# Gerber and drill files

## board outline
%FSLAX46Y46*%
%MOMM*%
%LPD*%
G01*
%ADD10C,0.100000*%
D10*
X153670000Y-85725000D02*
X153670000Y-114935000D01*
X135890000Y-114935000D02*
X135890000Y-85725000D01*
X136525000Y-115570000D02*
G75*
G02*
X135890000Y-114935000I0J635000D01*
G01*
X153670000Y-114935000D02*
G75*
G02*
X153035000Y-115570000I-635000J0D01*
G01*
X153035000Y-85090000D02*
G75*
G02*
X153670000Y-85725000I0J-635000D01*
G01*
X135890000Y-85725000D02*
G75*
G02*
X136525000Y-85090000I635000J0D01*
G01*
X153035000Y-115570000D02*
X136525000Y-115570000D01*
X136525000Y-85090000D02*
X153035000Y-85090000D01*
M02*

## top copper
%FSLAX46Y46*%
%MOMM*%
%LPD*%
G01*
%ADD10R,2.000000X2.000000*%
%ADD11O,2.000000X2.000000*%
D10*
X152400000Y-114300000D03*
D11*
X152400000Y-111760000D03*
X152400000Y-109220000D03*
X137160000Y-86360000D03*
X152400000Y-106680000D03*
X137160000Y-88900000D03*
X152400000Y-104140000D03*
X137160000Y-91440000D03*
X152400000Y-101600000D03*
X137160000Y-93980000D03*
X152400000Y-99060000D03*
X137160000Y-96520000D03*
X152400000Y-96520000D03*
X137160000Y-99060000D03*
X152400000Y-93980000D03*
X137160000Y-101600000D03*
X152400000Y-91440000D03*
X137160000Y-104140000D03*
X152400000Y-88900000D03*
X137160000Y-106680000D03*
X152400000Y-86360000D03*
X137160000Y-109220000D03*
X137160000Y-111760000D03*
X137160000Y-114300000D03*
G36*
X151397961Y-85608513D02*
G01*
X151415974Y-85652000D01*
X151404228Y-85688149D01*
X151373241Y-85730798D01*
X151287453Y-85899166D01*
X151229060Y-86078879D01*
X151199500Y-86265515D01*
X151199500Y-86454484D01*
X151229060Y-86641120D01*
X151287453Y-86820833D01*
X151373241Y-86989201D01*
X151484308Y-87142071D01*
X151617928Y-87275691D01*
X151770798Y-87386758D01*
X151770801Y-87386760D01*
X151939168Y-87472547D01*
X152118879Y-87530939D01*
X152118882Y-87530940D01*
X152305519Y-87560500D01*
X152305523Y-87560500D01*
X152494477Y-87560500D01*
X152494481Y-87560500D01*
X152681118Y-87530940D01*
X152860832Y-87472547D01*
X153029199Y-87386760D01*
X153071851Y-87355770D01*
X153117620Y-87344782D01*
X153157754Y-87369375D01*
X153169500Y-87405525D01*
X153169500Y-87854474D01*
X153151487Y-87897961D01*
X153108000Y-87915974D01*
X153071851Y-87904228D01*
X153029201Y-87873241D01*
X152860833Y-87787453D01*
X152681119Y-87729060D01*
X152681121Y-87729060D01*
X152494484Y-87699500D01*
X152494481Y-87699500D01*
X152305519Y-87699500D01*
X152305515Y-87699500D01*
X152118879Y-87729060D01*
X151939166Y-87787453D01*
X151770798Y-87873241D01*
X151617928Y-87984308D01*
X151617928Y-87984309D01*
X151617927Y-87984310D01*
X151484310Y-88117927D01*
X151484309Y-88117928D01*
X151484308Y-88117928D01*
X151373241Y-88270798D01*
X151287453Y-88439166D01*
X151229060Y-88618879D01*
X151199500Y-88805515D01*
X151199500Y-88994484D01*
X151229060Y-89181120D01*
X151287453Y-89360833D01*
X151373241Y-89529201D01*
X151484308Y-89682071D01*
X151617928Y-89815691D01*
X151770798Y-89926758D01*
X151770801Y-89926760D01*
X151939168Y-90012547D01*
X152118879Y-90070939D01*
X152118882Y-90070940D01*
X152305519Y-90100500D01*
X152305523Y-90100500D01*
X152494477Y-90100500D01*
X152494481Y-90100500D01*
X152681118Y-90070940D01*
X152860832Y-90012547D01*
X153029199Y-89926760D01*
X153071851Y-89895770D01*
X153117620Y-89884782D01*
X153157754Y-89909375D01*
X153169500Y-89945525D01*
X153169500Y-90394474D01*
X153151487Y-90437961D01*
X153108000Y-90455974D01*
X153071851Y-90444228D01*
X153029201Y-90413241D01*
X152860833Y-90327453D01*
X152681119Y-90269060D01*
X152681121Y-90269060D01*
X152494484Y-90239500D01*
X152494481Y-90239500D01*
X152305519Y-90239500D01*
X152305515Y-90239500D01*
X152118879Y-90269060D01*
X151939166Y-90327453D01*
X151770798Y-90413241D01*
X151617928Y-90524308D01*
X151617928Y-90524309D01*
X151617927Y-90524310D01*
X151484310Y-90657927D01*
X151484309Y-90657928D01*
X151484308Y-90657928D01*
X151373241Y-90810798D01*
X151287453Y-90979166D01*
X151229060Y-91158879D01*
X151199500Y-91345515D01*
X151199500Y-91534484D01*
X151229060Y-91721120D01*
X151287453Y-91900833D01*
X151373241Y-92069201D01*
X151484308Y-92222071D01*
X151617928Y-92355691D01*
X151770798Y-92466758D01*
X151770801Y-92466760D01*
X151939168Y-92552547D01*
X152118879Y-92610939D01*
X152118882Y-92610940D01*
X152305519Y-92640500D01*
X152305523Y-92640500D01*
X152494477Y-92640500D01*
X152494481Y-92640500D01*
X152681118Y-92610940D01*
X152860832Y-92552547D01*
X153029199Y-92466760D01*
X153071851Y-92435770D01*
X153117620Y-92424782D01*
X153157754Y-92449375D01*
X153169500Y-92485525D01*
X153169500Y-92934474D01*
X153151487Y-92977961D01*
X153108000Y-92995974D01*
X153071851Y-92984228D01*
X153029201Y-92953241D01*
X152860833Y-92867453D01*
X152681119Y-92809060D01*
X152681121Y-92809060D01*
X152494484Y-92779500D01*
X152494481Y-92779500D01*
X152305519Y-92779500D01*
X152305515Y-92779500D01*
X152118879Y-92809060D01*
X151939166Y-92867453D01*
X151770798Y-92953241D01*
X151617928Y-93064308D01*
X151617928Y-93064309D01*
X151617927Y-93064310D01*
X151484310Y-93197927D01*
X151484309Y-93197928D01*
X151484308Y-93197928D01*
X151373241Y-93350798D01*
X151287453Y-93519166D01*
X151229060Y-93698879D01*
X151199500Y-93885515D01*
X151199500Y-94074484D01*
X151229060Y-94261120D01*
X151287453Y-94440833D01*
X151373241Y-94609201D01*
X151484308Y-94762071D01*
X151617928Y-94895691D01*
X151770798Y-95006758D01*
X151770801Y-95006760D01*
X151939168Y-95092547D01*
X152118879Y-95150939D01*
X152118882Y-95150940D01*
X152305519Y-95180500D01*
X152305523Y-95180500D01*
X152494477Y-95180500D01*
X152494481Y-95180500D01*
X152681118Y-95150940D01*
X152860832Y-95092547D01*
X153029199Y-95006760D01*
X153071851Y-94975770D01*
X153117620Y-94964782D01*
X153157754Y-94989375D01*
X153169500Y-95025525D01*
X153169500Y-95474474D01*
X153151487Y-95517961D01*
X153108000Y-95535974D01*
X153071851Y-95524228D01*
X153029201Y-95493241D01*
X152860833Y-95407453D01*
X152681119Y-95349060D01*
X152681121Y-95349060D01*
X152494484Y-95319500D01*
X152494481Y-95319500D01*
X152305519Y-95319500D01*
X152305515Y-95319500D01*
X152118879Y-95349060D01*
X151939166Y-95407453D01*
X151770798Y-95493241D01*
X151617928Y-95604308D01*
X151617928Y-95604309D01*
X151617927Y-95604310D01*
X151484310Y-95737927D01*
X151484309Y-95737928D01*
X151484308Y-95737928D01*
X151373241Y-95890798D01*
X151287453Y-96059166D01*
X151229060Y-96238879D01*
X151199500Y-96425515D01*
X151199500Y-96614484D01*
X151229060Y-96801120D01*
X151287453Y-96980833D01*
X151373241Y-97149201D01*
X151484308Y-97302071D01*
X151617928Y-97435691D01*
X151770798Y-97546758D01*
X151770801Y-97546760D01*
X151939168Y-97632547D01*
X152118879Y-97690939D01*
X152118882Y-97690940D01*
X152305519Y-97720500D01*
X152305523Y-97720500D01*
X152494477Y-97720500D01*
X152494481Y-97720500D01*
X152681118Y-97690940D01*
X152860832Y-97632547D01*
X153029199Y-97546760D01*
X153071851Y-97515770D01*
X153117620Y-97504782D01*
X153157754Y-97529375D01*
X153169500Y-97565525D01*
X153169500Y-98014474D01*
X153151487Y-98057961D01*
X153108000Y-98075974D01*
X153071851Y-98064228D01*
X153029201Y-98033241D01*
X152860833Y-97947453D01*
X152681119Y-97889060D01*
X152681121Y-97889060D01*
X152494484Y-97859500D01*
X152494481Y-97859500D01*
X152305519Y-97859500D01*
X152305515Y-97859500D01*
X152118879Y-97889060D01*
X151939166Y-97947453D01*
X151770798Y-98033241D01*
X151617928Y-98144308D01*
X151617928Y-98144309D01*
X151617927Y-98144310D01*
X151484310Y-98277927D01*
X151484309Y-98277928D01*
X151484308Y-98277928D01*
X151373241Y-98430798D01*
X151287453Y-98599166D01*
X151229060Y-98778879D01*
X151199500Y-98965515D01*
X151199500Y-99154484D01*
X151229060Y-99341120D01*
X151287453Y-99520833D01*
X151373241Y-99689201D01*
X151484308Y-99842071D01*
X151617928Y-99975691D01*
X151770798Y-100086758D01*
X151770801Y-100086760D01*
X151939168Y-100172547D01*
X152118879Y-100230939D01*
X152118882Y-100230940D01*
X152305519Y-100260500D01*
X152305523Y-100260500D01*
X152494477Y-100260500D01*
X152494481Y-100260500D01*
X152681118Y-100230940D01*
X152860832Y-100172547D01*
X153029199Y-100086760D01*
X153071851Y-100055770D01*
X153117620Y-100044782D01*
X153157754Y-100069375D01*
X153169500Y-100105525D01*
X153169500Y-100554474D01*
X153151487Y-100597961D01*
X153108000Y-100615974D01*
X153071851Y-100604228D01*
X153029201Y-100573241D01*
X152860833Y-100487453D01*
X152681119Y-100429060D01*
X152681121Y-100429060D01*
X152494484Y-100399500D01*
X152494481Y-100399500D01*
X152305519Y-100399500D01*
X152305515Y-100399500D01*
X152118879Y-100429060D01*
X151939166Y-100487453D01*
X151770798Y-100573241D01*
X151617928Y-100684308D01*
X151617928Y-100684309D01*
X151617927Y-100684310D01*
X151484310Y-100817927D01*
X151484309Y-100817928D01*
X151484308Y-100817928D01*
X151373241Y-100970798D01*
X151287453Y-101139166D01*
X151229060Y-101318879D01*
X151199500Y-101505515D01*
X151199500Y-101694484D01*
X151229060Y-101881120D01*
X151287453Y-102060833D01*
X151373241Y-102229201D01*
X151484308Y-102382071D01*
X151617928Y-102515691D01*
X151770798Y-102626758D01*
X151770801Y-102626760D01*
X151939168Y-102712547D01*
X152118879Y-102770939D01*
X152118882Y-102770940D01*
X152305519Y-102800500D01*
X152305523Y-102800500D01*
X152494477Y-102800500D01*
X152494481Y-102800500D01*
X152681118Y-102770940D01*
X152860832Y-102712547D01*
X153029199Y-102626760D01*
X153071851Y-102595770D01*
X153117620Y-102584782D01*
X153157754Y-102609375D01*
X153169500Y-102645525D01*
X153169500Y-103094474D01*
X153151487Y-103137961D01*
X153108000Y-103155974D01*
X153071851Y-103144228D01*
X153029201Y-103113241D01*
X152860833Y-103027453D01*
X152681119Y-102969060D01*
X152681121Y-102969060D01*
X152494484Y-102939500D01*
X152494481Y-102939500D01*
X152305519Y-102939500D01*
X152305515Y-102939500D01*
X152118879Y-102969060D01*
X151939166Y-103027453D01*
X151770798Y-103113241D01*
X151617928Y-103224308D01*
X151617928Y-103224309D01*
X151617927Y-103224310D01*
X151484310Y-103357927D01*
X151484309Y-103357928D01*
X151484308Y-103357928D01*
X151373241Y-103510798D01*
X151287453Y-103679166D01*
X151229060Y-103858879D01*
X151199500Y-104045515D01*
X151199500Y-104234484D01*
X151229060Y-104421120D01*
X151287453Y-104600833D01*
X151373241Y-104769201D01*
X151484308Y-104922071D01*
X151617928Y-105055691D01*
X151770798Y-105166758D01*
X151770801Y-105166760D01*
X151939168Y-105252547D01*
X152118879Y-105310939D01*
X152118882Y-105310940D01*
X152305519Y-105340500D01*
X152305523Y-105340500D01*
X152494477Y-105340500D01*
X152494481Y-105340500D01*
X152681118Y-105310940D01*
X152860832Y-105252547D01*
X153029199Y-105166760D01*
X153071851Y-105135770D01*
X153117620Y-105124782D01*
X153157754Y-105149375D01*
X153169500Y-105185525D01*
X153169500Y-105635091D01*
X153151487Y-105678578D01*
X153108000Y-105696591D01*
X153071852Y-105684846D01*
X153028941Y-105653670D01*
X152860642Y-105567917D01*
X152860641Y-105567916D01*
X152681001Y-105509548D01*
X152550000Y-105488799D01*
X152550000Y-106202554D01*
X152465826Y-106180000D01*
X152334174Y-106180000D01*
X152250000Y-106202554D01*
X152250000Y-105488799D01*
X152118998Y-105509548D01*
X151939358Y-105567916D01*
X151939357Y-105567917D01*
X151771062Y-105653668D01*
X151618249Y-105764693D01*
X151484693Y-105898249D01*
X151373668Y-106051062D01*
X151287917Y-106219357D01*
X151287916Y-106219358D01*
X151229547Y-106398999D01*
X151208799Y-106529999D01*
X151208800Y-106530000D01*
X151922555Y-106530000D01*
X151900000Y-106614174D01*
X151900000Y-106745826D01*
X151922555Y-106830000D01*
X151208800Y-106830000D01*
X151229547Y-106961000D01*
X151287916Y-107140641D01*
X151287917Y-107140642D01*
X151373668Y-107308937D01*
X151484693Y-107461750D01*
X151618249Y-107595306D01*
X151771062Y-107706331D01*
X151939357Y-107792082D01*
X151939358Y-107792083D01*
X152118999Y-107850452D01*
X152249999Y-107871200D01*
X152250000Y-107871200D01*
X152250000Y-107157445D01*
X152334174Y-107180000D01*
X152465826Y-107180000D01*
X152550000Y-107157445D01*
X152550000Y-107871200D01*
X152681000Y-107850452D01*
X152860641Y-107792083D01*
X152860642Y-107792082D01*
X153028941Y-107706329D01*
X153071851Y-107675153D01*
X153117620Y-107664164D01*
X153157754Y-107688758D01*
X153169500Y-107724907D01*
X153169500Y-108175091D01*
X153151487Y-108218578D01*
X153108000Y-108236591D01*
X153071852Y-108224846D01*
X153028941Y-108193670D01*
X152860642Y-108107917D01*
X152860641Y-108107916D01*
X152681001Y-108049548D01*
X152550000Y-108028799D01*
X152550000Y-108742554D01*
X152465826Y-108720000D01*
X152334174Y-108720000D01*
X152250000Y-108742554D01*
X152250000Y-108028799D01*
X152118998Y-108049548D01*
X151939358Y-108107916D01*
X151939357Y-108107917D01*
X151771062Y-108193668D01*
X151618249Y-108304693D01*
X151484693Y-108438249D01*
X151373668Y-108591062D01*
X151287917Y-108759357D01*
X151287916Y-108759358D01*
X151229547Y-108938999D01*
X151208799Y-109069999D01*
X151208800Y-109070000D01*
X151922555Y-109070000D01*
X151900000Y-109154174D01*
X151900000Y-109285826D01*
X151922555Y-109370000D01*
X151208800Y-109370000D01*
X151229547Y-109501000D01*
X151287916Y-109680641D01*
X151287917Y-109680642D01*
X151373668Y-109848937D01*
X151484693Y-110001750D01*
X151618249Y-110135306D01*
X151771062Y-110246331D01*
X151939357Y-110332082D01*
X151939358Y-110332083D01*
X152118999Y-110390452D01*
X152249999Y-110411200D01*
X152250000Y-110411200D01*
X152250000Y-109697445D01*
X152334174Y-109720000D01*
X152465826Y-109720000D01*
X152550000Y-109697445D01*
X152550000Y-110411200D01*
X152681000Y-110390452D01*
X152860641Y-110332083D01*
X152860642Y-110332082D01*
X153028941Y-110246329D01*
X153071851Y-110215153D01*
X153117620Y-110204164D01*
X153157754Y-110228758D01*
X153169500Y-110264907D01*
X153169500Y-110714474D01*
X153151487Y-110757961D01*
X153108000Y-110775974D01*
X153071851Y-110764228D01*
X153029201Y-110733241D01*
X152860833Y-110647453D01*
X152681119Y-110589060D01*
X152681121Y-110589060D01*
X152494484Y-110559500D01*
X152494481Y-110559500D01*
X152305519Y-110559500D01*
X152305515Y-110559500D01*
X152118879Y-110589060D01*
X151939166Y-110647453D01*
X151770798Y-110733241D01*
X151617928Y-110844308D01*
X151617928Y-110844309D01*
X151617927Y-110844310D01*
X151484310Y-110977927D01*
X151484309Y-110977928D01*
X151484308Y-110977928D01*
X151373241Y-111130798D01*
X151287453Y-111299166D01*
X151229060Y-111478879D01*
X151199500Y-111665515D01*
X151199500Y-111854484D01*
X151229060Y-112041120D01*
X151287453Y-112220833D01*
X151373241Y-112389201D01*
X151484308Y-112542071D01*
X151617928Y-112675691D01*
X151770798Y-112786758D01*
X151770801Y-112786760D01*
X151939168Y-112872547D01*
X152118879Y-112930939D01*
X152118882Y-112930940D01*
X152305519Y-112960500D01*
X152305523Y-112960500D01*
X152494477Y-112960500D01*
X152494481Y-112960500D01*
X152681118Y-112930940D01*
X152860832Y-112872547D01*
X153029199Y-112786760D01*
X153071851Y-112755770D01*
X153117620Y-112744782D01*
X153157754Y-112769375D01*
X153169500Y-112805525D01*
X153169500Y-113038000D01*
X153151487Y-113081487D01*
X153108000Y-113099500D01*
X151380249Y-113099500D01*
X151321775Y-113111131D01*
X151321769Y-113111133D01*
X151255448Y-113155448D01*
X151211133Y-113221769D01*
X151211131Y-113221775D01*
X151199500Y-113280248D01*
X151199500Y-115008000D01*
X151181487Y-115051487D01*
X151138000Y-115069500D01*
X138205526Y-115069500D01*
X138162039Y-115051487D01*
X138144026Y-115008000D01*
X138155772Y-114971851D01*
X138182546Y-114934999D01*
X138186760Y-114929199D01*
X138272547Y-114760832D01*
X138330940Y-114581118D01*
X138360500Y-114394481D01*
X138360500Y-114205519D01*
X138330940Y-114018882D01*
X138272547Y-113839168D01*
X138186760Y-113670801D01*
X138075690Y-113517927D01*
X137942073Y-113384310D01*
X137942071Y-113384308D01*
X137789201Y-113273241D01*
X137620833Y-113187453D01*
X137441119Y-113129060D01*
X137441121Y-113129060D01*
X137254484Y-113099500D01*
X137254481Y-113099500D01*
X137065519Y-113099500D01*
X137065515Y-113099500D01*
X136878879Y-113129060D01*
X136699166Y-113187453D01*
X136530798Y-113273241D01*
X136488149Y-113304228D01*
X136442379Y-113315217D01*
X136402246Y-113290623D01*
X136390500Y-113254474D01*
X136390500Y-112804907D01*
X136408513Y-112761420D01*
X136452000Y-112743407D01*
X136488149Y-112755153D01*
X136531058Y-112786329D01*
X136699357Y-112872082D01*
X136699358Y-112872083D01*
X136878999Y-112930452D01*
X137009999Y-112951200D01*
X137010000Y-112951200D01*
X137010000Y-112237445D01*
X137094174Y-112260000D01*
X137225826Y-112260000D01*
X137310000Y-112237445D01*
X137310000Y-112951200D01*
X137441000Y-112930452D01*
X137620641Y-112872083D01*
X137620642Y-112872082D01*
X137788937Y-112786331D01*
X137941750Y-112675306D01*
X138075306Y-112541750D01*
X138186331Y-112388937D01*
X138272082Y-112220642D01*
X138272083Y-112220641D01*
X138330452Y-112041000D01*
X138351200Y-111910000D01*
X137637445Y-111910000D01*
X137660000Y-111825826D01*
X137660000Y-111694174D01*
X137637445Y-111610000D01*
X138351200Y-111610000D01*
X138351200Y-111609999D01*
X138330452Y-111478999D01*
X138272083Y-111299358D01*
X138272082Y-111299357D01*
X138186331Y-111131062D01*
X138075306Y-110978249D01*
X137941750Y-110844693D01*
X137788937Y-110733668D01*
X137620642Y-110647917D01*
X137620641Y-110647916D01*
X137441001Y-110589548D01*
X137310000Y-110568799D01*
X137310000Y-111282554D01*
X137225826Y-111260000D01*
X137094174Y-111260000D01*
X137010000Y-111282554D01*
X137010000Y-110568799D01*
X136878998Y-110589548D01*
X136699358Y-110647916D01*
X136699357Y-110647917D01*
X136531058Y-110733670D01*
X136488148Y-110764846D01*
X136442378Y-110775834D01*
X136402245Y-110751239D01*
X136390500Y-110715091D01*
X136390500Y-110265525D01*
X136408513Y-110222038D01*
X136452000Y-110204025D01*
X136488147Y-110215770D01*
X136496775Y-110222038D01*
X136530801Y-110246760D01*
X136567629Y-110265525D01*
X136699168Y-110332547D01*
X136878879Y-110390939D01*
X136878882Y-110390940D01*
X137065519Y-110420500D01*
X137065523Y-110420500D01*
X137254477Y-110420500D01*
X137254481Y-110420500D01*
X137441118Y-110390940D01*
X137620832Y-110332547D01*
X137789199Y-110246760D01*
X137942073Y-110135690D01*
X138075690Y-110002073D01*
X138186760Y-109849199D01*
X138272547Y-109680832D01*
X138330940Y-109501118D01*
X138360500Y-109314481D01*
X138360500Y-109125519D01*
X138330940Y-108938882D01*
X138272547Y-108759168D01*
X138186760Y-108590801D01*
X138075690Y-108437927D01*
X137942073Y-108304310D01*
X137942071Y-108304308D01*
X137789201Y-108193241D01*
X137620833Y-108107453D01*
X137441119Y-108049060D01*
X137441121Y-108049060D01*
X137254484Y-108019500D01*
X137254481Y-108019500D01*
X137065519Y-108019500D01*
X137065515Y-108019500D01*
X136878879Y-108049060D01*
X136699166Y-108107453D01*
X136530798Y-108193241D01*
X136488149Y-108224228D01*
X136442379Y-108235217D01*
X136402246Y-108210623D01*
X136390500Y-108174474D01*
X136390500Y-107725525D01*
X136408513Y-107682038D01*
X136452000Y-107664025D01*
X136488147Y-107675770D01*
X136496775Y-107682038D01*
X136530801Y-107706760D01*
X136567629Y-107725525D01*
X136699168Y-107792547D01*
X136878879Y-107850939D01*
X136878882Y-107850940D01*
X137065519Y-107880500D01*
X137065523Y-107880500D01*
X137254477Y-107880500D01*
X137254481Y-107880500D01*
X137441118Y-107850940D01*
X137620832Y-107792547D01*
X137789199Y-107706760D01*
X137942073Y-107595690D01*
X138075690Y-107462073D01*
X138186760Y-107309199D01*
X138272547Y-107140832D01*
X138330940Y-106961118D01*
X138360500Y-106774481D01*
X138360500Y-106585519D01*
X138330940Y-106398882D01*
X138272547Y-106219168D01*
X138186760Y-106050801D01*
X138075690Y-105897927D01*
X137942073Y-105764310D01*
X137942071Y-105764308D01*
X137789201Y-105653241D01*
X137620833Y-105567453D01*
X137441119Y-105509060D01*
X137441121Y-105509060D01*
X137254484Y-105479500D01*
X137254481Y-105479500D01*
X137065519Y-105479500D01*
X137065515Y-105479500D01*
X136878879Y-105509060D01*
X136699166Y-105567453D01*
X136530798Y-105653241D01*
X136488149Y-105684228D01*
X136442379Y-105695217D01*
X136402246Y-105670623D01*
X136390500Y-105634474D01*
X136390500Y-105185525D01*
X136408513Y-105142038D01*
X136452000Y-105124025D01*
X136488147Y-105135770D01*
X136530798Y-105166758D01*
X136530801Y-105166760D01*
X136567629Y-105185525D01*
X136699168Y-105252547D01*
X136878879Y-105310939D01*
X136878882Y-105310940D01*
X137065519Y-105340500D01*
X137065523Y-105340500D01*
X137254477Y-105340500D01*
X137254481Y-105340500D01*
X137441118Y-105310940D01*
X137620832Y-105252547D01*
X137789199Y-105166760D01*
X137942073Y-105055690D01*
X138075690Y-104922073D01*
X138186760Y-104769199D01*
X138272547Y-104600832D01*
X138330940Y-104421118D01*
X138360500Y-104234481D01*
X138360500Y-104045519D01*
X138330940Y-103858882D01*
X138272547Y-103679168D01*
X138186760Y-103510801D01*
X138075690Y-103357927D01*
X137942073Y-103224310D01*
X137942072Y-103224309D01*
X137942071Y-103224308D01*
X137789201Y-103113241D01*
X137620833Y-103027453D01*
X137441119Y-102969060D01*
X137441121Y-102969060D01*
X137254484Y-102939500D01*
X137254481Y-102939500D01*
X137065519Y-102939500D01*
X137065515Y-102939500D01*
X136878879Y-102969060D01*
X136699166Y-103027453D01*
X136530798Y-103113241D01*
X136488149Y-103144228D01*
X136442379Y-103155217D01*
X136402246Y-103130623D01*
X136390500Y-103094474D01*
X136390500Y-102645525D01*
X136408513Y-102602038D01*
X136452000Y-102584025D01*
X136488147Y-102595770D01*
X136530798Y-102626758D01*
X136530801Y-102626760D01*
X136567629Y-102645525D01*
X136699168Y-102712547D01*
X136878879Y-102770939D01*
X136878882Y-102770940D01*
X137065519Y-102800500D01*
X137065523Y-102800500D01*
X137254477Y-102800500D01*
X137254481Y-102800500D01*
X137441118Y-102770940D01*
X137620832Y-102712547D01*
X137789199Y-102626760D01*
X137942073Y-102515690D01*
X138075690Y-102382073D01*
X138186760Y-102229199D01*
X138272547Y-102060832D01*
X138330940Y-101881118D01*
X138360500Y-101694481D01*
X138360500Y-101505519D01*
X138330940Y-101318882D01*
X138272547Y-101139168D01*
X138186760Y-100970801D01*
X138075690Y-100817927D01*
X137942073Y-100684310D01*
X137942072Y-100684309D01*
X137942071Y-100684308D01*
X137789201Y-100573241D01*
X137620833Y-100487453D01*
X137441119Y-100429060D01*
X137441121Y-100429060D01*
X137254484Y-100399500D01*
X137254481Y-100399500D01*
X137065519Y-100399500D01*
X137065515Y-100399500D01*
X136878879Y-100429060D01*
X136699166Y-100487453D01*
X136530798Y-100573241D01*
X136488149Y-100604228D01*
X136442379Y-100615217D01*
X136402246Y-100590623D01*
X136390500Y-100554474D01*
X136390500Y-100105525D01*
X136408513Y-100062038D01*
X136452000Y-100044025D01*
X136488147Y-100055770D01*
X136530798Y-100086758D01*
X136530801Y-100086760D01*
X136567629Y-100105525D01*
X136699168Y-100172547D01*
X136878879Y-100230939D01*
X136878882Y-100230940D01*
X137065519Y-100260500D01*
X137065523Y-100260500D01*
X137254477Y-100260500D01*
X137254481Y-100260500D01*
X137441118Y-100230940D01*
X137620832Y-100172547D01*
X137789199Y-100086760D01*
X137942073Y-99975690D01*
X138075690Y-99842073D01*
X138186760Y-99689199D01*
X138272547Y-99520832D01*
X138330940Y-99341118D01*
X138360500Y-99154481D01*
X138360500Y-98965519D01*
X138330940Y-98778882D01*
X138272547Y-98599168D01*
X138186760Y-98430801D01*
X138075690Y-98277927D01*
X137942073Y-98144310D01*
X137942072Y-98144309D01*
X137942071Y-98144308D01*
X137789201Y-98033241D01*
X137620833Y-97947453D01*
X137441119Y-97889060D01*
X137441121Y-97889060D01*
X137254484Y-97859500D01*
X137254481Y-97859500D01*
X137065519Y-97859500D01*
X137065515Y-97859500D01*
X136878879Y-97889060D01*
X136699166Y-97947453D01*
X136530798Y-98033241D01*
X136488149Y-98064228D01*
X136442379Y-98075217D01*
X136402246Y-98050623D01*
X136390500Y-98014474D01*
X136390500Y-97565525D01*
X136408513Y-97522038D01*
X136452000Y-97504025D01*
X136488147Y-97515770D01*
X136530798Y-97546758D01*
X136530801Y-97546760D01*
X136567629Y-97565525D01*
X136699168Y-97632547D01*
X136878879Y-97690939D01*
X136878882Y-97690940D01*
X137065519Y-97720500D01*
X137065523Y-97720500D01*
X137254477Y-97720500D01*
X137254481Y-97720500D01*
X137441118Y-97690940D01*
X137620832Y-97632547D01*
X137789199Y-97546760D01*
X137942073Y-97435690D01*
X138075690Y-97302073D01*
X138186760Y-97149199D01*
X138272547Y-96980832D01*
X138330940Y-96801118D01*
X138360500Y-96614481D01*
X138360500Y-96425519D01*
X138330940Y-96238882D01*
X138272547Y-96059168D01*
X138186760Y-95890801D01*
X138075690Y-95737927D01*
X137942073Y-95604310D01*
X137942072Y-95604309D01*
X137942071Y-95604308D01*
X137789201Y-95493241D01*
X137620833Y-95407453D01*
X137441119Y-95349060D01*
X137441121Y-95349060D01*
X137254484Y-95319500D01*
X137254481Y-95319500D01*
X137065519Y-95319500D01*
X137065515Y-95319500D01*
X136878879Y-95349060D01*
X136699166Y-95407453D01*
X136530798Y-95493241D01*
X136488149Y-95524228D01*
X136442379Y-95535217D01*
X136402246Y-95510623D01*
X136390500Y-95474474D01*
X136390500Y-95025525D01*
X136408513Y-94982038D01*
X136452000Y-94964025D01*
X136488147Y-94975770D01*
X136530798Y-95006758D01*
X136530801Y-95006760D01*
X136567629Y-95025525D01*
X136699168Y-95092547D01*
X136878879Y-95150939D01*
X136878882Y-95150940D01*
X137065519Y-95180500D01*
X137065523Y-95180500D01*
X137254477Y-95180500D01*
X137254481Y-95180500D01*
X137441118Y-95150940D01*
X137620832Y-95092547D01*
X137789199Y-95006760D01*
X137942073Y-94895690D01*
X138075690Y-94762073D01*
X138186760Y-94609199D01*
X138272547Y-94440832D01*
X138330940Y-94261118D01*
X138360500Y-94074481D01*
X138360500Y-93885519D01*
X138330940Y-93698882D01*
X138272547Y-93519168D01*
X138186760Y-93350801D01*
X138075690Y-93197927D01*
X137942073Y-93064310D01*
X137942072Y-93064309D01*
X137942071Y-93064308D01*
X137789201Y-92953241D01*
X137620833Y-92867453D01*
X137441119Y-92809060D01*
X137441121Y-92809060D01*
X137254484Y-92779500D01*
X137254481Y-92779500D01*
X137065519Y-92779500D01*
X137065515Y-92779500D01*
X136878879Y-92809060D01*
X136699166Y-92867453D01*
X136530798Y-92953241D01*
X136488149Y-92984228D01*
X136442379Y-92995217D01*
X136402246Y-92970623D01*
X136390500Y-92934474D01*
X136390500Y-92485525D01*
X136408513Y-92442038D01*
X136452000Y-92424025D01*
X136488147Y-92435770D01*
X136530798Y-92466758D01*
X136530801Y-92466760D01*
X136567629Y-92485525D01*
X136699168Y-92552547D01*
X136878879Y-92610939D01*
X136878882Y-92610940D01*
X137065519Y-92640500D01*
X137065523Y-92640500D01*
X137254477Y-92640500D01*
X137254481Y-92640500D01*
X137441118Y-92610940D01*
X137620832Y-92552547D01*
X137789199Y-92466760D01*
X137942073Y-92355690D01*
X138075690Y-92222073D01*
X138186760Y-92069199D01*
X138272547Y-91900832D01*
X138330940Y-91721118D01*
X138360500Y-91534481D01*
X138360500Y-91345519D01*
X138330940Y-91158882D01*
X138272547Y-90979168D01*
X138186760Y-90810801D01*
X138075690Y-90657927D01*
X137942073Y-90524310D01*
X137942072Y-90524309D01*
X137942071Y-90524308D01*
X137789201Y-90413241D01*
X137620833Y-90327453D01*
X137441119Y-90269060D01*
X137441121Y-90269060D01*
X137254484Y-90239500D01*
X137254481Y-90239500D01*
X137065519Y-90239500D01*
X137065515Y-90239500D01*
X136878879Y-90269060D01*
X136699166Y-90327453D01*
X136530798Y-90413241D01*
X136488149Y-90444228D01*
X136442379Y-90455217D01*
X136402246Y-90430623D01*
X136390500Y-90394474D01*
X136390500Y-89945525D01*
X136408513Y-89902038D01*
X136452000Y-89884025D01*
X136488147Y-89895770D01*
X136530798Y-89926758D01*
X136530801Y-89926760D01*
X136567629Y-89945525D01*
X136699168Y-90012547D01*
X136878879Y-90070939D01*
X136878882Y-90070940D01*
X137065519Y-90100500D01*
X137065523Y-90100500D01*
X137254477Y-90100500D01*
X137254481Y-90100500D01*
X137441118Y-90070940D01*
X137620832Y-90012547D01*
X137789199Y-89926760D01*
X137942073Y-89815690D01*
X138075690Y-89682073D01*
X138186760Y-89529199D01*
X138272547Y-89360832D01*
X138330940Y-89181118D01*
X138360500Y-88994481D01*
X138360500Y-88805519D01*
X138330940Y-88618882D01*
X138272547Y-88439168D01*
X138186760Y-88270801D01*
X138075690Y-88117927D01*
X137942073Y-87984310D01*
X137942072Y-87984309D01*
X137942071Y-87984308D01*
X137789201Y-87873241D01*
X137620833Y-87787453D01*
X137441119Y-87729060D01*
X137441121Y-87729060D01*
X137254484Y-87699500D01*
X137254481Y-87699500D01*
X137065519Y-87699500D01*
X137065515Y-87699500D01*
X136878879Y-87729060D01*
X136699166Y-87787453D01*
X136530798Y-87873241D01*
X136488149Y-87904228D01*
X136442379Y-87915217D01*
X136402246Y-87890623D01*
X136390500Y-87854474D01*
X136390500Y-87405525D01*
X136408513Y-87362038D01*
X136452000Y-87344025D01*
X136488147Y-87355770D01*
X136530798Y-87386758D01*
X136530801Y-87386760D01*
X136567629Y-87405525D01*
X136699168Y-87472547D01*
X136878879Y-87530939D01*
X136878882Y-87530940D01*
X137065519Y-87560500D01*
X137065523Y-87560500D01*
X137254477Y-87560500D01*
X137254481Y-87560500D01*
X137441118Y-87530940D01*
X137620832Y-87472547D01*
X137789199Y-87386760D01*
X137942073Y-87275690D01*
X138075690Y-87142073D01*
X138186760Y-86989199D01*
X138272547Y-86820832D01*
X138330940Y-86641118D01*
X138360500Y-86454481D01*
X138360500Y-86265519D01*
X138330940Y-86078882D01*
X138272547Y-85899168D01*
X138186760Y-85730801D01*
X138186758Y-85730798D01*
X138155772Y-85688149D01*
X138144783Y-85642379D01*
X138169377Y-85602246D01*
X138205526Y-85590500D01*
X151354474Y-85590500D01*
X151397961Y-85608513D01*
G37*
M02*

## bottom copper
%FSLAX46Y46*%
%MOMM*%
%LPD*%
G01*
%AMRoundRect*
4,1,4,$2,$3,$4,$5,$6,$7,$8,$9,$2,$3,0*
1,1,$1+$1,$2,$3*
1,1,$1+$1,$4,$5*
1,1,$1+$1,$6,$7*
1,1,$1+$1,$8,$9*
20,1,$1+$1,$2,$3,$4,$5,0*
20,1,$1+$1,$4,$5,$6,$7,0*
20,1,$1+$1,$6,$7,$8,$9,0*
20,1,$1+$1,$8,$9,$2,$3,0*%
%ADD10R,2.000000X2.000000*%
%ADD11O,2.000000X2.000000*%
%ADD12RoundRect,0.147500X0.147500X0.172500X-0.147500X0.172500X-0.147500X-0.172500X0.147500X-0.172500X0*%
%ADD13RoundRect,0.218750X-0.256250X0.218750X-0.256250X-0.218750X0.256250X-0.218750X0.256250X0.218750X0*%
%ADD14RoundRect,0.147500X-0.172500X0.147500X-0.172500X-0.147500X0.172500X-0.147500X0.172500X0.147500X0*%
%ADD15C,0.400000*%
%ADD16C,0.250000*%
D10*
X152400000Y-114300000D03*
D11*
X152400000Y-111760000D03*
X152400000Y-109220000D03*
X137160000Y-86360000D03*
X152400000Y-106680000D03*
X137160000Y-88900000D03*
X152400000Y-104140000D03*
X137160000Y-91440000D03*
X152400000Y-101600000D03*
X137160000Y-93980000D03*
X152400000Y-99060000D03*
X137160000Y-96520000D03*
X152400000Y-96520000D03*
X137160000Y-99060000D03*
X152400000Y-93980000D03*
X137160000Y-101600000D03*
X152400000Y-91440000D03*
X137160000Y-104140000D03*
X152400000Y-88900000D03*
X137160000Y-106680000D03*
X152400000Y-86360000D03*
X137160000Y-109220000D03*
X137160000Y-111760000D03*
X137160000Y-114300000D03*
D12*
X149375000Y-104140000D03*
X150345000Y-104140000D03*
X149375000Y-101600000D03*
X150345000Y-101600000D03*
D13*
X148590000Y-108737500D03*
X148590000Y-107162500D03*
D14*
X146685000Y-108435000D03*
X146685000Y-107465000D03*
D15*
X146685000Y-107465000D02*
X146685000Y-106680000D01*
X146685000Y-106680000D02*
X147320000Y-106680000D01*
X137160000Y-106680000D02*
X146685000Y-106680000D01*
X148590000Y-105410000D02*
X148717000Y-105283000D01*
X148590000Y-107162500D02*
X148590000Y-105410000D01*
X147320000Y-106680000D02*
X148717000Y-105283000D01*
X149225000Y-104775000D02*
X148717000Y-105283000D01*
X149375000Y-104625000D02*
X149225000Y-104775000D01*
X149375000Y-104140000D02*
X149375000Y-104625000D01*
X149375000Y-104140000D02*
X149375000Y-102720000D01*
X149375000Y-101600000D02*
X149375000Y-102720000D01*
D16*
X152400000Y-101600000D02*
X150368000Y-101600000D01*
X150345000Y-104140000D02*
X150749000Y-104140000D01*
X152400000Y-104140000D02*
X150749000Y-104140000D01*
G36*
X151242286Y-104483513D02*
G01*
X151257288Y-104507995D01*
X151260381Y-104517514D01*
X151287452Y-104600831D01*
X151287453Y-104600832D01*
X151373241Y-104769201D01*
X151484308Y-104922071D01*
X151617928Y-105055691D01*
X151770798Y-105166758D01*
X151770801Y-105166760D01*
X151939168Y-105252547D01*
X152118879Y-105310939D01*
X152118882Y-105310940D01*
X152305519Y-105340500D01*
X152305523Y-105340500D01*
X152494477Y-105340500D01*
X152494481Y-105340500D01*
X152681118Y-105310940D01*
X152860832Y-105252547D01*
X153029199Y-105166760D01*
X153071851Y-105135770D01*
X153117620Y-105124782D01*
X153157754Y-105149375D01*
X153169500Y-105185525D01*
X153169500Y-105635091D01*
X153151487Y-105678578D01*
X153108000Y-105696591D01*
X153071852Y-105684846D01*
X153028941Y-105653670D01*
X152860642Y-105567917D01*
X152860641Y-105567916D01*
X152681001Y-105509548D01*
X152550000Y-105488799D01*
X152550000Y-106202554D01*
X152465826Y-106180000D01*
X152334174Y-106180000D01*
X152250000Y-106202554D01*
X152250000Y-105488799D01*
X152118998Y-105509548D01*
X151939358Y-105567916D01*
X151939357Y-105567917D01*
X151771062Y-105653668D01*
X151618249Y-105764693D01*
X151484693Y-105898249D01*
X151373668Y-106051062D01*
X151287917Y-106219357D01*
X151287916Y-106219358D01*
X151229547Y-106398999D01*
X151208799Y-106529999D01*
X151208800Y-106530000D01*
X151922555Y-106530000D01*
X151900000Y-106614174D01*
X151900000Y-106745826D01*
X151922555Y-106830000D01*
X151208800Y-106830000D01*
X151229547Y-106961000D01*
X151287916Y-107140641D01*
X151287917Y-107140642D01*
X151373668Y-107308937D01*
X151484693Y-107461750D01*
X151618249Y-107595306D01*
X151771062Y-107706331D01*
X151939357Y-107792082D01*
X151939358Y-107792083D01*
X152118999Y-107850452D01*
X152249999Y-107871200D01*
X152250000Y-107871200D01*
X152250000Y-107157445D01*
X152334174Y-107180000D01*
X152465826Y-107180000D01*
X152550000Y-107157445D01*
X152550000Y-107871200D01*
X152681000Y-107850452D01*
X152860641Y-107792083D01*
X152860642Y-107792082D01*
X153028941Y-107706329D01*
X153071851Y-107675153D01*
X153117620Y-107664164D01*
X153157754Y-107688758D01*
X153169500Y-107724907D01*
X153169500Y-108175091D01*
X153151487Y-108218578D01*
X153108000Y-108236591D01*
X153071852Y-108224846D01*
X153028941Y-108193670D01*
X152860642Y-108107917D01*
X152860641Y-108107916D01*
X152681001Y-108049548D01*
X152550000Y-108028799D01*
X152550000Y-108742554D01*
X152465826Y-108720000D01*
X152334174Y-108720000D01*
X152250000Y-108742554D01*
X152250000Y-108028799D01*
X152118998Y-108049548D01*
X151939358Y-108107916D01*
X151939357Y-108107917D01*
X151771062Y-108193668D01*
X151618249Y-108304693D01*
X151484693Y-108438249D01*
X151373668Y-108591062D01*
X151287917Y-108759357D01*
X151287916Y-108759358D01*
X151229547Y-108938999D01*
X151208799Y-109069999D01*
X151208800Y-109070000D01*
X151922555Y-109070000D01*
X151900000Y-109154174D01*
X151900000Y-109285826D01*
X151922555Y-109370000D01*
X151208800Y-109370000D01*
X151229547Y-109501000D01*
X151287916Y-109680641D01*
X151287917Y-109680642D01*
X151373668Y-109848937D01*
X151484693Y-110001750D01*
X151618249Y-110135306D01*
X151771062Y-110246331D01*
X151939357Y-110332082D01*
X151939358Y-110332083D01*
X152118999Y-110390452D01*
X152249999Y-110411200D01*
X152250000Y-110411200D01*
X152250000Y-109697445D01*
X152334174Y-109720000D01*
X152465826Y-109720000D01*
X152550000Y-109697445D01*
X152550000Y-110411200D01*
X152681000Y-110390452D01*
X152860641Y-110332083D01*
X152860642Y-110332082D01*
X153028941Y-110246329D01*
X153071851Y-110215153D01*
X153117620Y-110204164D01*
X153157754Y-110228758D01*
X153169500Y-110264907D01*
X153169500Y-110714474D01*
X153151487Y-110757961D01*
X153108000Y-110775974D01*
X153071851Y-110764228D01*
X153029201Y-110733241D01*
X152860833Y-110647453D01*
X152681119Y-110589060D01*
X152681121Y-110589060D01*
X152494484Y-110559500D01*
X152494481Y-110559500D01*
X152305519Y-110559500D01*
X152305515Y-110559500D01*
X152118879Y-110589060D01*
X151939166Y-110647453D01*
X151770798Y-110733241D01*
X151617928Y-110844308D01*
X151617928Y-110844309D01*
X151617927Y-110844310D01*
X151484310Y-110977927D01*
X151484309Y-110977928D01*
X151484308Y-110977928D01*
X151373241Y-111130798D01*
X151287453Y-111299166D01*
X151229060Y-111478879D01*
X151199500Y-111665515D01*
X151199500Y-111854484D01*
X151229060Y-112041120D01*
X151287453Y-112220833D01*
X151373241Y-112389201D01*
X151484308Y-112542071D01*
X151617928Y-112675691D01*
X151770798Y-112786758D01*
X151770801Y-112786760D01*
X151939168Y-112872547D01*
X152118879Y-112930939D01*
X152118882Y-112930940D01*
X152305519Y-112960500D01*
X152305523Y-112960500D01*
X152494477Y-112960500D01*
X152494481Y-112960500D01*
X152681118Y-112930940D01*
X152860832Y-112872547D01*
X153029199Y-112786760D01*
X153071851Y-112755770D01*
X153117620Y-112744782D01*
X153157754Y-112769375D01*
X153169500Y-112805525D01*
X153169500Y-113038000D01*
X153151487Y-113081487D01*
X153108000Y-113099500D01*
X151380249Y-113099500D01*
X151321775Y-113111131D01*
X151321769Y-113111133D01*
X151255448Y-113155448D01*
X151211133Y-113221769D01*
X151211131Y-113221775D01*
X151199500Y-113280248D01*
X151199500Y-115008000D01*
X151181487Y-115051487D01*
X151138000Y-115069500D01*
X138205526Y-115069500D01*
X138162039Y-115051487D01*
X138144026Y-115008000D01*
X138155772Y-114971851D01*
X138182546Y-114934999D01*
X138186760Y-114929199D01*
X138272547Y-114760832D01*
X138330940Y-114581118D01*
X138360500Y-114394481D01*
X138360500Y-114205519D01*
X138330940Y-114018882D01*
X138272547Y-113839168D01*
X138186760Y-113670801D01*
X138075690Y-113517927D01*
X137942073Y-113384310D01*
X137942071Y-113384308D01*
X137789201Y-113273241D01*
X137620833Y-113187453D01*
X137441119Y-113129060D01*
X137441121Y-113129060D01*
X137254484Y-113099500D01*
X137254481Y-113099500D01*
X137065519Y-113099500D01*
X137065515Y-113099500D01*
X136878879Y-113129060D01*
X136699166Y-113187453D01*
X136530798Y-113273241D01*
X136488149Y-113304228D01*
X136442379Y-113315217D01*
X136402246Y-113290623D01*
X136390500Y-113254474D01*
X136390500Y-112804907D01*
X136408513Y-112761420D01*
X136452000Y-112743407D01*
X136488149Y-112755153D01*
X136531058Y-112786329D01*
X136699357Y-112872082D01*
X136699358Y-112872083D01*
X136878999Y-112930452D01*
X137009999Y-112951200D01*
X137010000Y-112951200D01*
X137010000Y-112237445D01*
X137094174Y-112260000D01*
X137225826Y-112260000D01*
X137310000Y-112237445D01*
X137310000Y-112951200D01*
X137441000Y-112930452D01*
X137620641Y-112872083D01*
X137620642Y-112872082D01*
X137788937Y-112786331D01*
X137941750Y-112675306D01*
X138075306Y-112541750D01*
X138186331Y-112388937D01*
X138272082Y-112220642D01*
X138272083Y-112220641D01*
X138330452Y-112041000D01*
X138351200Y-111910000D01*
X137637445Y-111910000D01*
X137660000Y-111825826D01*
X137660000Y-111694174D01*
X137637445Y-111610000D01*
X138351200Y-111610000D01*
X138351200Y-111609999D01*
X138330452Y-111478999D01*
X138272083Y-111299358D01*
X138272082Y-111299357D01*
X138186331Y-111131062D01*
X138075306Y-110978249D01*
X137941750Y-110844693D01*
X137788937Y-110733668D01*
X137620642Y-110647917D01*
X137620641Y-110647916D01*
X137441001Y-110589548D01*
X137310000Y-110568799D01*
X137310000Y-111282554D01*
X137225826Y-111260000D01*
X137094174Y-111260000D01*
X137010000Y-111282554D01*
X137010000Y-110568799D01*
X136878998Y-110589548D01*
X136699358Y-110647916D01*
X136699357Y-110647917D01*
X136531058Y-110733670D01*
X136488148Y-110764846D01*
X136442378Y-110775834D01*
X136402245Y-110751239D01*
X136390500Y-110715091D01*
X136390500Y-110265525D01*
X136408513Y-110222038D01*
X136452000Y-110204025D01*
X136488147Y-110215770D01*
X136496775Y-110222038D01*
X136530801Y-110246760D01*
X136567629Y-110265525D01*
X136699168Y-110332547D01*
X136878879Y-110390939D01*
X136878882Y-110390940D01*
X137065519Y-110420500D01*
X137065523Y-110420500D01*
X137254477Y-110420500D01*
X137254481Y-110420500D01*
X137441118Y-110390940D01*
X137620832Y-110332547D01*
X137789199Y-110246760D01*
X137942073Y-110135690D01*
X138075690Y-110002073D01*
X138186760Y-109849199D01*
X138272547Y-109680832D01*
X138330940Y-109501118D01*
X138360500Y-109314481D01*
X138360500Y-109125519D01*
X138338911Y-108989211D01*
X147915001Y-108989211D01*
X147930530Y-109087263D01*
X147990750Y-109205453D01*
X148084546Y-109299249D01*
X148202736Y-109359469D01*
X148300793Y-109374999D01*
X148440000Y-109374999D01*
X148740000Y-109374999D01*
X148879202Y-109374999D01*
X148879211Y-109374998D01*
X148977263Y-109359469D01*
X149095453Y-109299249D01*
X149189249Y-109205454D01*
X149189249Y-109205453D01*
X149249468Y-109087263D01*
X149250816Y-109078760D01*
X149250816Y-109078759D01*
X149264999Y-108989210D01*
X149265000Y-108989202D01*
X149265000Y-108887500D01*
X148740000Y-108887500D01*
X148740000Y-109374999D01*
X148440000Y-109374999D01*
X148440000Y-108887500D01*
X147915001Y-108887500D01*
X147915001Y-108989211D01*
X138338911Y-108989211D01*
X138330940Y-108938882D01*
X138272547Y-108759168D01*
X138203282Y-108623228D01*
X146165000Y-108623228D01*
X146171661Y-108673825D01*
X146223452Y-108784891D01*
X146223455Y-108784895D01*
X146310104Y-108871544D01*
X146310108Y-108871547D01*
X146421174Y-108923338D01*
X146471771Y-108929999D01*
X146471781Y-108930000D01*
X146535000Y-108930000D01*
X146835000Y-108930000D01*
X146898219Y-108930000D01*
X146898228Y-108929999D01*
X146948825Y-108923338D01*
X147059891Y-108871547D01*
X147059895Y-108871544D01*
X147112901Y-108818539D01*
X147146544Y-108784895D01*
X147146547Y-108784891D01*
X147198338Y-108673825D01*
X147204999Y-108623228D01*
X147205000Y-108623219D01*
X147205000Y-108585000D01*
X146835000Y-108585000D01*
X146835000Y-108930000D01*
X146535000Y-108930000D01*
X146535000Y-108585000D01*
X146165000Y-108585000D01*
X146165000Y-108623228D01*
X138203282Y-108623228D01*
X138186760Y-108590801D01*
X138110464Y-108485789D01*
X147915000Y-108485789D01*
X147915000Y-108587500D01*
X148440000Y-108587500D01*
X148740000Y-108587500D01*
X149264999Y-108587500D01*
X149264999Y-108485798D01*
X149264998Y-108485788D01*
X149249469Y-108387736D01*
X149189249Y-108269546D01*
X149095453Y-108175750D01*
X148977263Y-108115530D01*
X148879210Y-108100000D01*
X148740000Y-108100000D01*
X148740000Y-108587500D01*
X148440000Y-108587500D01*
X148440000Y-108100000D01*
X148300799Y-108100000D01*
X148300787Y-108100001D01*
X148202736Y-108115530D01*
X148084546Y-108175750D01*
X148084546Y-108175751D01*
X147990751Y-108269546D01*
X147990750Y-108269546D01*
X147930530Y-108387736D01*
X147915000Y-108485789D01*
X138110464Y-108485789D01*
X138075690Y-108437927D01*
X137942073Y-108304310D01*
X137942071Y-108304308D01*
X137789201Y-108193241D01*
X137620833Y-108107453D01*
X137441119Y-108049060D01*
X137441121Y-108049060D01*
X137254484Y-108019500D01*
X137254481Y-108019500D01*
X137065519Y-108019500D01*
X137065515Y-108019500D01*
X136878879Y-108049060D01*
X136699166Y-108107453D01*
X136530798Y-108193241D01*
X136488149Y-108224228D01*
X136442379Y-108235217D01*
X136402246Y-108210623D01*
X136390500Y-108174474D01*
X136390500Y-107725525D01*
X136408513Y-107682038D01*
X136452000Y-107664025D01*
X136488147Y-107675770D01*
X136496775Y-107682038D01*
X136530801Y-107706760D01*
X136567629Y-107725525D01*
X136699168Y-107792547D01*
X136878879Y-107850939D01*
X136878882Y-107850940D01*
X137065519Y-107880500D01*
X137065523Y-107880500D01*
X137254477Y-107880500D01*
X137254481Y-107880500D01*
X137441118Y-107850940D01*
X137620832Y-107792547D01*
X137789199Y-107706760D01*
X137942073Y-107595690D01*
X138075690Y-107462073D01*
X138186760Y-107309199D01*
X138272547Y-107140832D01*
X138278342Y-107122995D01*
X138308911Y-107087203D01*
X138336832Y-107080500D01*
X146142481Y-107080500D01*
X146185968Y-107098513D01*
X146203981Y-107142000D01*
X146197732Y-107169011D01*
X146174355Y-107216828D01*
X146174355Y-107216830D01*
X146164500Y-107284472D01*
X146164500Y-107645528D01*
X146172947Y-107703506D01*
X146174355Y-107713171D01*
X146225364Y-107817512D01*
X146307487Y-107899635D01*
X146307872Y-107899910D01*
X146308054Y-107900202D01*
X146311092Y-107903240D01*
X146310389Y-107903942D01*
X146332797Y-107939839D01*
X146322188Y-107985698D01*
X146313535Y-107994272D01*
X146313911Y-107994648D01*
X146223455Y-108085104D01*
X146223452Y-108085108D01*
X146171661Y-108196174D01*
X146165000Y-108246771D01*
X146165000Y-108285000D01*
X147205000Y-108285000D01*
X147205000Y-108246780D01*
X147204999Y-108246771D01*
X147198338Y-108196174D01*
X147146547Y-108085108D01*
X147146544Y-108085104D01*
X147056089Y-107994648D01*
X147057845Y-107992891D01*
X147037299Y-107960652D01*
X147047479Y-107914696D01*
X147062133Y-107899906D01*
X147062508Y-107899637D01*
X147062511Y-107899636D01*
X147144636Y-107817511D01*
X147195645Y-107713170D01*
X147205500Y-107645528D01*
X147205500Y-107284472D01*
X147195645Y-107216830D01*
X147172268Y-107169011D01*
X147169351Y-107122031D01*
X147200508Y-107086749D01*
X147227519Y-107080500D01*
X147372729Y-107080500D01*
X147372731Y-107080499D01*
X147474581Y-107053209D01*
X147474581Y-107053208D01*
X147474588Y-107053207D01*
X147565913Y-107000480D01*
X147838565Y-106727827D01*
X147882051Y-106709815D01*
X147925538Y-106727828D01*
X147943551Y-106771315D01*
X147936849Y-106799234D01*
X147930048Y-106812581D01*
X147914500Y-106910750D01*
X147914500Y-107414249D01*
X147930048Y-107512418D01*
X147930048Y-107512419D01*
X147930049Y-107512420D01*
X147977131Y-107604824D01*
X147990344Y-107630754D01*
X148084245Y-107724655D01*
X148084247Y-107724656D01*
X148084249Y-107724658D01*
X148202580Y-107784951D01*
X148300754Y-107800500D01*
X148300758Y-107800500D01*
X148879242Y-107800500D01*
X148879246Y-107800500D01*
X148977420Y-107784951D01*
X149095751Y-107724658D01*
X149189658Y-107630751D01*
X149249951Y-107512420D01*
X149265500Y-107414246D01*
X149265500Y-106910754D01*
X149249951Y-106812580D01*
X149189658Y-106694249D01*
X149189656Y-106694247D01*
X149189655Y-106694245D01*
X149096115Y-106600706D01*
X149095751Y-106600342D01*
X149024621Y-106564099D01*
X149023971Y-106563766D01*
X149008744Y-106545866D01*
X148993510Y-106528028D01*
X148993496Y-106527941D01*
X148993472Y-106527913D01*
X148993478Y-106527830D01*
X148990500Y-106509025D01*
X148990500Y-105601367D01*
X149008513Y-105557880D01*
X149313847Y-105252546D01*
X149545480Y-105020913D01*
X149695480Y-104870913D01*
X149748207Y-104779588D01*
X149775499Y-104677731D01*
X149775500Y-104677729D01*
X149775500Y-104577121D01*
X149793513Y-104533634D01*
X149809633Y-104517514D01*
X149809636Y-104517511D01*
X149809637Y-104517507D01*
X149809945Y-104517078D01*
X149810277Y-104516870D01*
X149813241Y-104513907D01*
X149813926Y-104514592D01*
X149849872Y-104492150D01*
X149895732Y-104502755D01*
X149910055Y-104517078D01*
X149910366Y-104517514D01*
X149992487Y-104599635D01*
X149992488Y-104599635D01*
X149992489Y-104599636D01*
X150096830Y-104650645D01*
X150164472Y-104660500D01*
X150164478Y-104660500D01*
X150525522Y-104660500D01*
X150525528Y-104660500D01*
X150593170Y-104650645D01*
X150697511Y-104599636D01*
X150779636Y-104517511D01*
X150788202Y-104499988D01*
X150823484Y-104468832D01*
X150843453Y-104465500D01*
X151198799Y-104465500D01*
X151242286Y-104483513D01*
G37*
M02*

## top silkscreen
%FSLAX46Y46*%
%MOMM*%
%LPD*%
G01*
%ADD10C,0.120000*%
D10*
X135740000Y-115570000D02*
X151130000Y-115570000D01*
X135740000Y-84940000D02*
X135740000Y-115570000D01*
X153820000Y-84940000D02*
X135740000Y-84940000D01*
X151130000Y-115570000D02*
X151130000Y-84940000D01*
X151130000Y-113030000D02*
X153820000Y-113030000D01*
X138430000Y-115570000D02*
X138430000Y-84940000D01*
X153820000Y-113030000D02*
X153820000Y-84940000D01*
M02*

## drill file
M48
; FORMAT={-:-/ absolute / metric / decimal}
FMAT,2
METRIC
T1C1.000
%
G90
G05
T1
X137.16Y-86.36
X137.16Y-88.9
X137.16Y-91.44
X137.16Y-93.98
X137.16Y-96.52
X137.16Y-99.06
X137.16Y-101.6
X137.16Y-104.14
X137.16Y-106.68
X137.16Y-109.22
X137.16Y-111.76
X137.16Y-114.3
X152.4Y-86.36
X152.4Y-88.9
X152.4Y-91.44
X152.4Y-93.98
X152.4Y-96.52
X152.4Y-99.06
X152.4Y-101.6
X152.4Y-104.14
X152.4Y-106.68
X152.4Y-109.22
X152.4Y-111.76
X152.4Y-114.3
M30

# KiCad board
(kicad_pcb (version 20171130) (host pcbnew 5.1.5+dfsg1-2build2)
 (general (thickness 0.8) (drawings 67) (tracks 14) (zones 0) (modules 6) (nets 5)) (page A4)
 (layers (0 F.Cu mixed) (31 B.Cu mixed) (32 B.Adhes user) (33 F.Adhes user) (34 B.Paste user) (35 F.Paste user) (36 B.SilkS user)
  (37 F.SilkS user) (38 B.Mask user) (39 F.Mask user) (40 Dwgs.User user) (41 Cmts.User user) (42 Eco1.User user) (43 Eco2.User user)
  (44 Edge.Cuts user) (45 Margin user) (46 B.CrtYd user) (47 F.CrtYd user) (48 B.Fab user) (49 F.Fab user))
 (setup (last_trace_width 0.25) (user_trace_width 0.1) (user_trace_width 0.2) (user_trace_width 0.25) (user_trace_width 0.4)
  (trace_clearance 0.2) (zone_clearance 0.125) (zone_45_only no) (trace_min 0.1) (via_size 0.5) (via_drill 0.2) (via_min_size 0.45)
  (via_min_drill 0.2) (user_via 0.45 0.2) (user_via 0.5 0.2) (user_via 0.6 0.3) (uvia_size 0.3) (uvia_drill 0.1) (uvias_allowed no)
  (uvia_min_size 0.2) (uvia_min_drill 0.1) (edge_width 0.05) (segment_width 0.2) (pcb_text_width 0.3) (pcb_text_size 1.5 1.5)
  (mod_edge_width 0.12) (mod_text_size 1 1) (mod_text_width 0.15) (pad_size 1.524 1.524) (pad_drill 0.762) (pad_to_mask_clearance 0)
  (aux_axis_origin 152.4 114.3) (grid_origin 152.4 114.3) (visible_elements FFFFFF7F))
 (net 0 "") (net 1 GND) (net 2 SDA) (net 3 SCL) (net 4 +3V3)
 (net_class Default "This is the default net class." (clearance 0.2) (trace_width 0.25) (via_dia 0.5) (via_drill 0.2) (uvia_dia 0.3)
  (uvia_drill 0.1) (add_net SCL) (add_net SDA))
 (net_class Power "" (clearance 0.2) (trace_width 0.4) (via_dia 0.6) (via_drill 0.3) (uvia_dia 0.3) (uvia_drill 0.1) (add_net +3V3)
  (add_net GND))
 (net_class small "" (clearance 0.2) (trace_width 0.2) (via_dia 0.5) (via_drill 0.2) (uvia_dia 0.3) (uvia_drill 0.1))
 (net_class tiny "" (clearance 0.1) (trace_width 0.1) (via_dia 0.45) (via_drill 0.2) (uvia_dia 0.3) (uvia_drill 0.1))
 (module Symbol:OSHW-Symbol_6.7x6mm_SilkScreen (layer B.Cu) (at 145.415 91.44 270)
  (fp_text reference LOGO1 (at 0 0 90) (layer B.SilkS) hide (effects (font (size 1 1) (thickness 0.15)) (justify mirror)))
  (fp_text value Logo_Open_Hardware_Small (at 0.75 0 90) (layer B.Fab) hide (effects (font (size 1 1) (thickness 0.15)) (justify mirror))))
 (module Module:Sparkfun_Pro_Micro (layer F.Cu) (at 152.4 114.3 180)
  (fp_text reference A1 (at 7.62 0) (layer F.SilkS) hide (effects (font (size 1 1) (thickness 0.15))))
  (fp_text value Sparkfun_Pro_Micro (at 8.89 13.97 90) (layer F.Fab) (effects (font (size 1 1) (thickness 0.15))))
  (fp_line (start 16.66 -1.27) (end 1.27 -1.27) (layer F.SilkS) (width 0.12))
  (fp_line (start 16.66 29.36) (end 16.66 -1.27) (layer F.SilkS) (width 0.12))
  (fp_line (start -1.42 29.36) (end 16.66 29.36) (layer F.SilkS) (width 0.12))
  (fp_line (start 1.27 -1.27) (end 1.27 29.36) (layer F.SilkS) (width 0.12))
  (fp_line (start 1.27 1.27) (end -1.42 1.27) (layer F.SilkS) (width 0.12))
  (fp_line (start 13.97 -1.27) (end 13.97 29.36) (layer F.SilkS) (width 0.12))
  (fp_line (start -1.42 1.27) (end -1.42 29.36) (layer F.SilkS) (width 0.12))
  (pad 1 thru_hole rect (at 0 0 180) (size 2 2) (drill 1) (layers *.Cu *.Mask))
  (pad 2 thru_hole oval (at 0 2.54 180) (size 2 2) (drill 1) (layers *.Cu *.Mask))
  (pad 3 thru_hole oval (at 0 5.08 180) (size 2 2) (drill 1) (layers *.Cu *.Mask) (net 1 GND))
  (pad 13 thru_hole oval (at 15.24 27.94 180) (size 2 2) (drill 1) (layers *.Cu *.Mask))
  (pad 4 thru_hole oval (at 0 7.62 180) (size 2 2) (drill 1) (layers *.Cu *.Mask) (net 1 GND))
  (pad 14 thru_hole oval (at 15.24 25.4 180) (size 2 2) (drill 1) (layers *.Cu *.Mask))
  (pad 5 thru_hole oval (at 0 10.16 180) (size 2 2) (drill 1) (layers *.Cu *.Mask) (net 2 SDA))
  (pad 15 thru_hole oval (at 15.24 22.86 180) (size 2 2) (drill 1) (layers *.Cu *.Mask))
  (pad 6 thru_hole oval (at 0 12.7 180) (size 2 2) (drill 1) (layers *.Cu *.Mask) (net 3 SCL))
  (pad 16 thru_hole oval (at 15.24 20.32 180) (size 2 2) (drill 1) (layers *.Cu *.Mask))
  (pad 7 thru_hole oval (at 0 15.24 180) (size 2 2) (drill 1) (layers *.Cu *.Mask))
  (pad 17 thru_hole oval (at 15.24 17.78 180) (size 2 2) (drill 1) (layers *.Cu *.Mask))
  (pad 8 thru_hole oval (at 0 17.78 180) (size 2 2) (drill 1) (layers *.Cu *.Mask))
  (pad 18 thru_hole oval (at 15.24 15.24 180) (size 2 2) (drill 1) (layers *.Cu *.Mask))
  (pad 9 thru_hole oval (at 0 20.32 180) (size 2 2) (drill 1) (layers *.Cu *.Mask))
  (pad 19 thru_hole oval (at 15.24 12.7 180) (size 2 2) (drill 1) (layers *.Cu *.Mask))
  (pad 10 thru_hole oval (at 0 22.86 180) (size 2 2) (drill 1) (layers *.Cu *.Mask))
  (pad 20 thru_hole oval (at 15.24 10.16 180) (size 2 2) (drill 1) (layers *.Cu *.Mask))
  (pad 11 thru_hole oval (at 0 25.4 180) (size 2 2) (drill 1) (layers *.Cu *.Mask))
  (pad 21 thru_hole oval (at 15.24 7.62 180) (size 2 2) (drill 1) (layers *.Cu *.Mask) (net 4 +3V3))
  (pad 12 thru_hole oval (at 0 27.94 180) (size 2 2) (drill 1) (layers *.Cu *.Mask))
  (pad 22 thru_hole oval (at 15.24 5.08 180) (size 2 2) (drill 1) (layers *.Cu *.Mask))
  (pad 23 thru_hole oval (at 15.24 2.54 180) (size 2 2) (drill 1) (layers *.Cu *.Mask) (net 1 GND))
  (pad 24 thru_hole oval (at 15.24 0 180) (size 2 2) (drill 1) (layers *.Cu *.Mask)))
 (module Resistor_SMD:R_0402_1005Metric (layer B.Cu) (at 149.86 104.14 180)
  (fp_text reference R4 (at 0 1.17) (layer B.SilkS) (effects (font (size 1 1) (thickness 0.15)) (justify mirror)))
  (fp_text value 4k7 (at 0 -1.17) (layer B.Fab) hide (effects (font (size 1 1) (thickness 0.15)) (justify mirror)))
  (pad 2 smd roundrect (at 0.485 0 180) (size 0.59 0.64) (layers B.Cu B.Paste B.Mask) (roundrect_rratio 0.25) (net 4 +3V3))
  (pad 1 smd roundrect (at -0.485 0 180) (size 0.59 0.64) (layers B.Cu B.Paste B.Mask) (roundrect_rratio 0.25) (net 2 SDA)))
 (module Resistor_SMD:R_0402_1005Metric (layer B.Cu) (at 149.86 101.6 180)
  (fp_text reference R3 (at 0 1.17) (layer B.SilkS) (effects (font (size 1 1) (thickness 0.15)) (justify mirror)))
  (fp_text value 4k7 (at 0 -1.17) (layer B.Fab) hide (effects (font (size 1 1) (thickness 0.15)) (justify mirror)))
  (pad 2 smd roundrect (at 0.485 0 180) (size 0.59 0.64) (layers B.Cu B.Paste B.Mask) (roundrect_rratio 0.25) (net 4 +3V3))
  (pad 1 smd roundrect (at -0.485 0 180) (size 0.59 0.64) (layers B.Cu B.Paste B.Mask) (roundrect_rratio 0.25) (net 3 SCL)))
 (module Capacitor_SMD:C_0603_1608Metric (layer B.Cu) (at 148.59 107.95 270)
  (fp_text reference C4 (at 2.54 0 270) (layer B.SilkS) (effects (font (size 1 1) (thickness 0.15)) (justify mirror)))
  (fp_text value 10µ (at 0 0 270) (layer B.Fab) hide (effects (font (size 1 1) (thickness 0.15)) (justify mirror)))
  (pad 2 smd roundrect (at 0.7875 0 270) (size 0.875 0.95) (layers B.Cu B.Paste B.Mask) (roundrect_rratio 0.25) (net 1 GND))
  (pad 1 smd roundrect (at -0.7875 0 270) (size 0.875 0.95) (layers B.Cu B.Paste B.Mask) (roundrect_rratio 0.25) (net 4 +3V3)))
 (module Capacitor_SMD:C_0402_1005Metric (layer B.Cu) (at 146.685 107.95 270)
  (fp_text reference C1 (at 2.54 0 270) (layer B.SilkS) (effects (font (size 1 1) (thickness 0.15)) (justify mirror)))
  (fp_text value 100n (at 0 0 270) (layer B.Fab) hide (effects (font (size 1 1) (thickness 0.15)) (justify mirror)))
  (pad 2 smd roundrect (at 0.485 0 270) (size 0.59 0.64) (layers B.Cu B.Paste B.Mask) (roundrect_rratio 0.25) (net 1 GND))
  (pad 1 smd roundrect (at -0.485 0 270) (size 0.59 0.64) (layers B.Cu B.Paste B.Mask) (roundrect_rratio 0.25) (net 4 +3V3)))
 (gr_line (start 153.67 85.725) (end 153.67 114.935) (layer Edge.Cuts) (width 0.1))
 (gr_line (start 135.89 114.935) (end 135.89 85.725) (layer Edge.Cuts) (width 0.1))
 (gr_arc (start 136.525 114.935) (end 135.89 114.935) (angle -90) (layer Edge.Cuts) (width 0.1))
 (gr_arc (start 153.035 114.935) (end 153.035 115.57) (angle -90) (layer Edge.Cuts) (width 0.1))
 (gr_arc (start 153.035 85.725) (end 153.67 85.725) (angle -90) (layer Edge.Cuts) (width 0.1))
 (gr_arc (start 136.525 85.725) (end 136.525 85.09) (angle -90) (layer Edge.Cuts) (width 0.1))
 (gr_line (start 153.035 115.57) (end 136.525 115.57) (layer Edge.Cuts) (width 0.1))
 (gr_line (start 136.525 85.09) (end 153.035 85.09) (layer Edge.Cuts) (width 0.1))
 (segment (start 146.685 107.465) (end 146.685 106.68) (width 0.4) (layer B.Cu) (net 4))
 (segment (start 146.685 106.68) (end 147.32 106.68) (width 0.4) (layer B.Cu) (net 4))
 (segment (start 137.16 106.68) (end 146.685 106.68) (width 0.4) (layer B.Cu) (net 4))
 (segment (start 148.59 105.41) (end 148.717 105.283) (width 0.4) (layer B.Cu) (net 4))
 (segment (start 148.59 107.1625) (end 148.59 105.41) (width 0.4) (layer B.Cu) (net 4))
 (segment (start 147.32 106.68) (end 148.717 105.283) (width 0.4) (layer B.Cu) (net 4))
 (segment (start 149.225 104.775) (end 148.717 105.283) (width 0.4) (layer B.Cu) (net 4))
 (segment (start 149.375 104.625) (end 149.225 104.775) (width 0.4) (layer B.Cu) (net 4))
 (segment (start 149.375 104.14) (end 149.375 104.625) (width 0.4) (layer B.Cu) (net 4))
 (segment (start 149.375 104.14) (end 149.375 102.72) (width 0.4) (layer B.Cu) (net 4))
 (segment (start 149.375 101.6) (end 149.375 102.72) (width 0.4) (layer B.Cu) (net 4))
 (segment (start 152.4 101.6) (end 150.368 101.6) (width 0.25) (layer B.Cu) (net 3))
 (segment (start 150.345 104.14) (end 150.749 104.14) (width 0.25) (layer B.Cu) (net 2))
 (segment (start 152.4 104.14) (end 150.749 104.14) (width 0.25) (layer B.Cu) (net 2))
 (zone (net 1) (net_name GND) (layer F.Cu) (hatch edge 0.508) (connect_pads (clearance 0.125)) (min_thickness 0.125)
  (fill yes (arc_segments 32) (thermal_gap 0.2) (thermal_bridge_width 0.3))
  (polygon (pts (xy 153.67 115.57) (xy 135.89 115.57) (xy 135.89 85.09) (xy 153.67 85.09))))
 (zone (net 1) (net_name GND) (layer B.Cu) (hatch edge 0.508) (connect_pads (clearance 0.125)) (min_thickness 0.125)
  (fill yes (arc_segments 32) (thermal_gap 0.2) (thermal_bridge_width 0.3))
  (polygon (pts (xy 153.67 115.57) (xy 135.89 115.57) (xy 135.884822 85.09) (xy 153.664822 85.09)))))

